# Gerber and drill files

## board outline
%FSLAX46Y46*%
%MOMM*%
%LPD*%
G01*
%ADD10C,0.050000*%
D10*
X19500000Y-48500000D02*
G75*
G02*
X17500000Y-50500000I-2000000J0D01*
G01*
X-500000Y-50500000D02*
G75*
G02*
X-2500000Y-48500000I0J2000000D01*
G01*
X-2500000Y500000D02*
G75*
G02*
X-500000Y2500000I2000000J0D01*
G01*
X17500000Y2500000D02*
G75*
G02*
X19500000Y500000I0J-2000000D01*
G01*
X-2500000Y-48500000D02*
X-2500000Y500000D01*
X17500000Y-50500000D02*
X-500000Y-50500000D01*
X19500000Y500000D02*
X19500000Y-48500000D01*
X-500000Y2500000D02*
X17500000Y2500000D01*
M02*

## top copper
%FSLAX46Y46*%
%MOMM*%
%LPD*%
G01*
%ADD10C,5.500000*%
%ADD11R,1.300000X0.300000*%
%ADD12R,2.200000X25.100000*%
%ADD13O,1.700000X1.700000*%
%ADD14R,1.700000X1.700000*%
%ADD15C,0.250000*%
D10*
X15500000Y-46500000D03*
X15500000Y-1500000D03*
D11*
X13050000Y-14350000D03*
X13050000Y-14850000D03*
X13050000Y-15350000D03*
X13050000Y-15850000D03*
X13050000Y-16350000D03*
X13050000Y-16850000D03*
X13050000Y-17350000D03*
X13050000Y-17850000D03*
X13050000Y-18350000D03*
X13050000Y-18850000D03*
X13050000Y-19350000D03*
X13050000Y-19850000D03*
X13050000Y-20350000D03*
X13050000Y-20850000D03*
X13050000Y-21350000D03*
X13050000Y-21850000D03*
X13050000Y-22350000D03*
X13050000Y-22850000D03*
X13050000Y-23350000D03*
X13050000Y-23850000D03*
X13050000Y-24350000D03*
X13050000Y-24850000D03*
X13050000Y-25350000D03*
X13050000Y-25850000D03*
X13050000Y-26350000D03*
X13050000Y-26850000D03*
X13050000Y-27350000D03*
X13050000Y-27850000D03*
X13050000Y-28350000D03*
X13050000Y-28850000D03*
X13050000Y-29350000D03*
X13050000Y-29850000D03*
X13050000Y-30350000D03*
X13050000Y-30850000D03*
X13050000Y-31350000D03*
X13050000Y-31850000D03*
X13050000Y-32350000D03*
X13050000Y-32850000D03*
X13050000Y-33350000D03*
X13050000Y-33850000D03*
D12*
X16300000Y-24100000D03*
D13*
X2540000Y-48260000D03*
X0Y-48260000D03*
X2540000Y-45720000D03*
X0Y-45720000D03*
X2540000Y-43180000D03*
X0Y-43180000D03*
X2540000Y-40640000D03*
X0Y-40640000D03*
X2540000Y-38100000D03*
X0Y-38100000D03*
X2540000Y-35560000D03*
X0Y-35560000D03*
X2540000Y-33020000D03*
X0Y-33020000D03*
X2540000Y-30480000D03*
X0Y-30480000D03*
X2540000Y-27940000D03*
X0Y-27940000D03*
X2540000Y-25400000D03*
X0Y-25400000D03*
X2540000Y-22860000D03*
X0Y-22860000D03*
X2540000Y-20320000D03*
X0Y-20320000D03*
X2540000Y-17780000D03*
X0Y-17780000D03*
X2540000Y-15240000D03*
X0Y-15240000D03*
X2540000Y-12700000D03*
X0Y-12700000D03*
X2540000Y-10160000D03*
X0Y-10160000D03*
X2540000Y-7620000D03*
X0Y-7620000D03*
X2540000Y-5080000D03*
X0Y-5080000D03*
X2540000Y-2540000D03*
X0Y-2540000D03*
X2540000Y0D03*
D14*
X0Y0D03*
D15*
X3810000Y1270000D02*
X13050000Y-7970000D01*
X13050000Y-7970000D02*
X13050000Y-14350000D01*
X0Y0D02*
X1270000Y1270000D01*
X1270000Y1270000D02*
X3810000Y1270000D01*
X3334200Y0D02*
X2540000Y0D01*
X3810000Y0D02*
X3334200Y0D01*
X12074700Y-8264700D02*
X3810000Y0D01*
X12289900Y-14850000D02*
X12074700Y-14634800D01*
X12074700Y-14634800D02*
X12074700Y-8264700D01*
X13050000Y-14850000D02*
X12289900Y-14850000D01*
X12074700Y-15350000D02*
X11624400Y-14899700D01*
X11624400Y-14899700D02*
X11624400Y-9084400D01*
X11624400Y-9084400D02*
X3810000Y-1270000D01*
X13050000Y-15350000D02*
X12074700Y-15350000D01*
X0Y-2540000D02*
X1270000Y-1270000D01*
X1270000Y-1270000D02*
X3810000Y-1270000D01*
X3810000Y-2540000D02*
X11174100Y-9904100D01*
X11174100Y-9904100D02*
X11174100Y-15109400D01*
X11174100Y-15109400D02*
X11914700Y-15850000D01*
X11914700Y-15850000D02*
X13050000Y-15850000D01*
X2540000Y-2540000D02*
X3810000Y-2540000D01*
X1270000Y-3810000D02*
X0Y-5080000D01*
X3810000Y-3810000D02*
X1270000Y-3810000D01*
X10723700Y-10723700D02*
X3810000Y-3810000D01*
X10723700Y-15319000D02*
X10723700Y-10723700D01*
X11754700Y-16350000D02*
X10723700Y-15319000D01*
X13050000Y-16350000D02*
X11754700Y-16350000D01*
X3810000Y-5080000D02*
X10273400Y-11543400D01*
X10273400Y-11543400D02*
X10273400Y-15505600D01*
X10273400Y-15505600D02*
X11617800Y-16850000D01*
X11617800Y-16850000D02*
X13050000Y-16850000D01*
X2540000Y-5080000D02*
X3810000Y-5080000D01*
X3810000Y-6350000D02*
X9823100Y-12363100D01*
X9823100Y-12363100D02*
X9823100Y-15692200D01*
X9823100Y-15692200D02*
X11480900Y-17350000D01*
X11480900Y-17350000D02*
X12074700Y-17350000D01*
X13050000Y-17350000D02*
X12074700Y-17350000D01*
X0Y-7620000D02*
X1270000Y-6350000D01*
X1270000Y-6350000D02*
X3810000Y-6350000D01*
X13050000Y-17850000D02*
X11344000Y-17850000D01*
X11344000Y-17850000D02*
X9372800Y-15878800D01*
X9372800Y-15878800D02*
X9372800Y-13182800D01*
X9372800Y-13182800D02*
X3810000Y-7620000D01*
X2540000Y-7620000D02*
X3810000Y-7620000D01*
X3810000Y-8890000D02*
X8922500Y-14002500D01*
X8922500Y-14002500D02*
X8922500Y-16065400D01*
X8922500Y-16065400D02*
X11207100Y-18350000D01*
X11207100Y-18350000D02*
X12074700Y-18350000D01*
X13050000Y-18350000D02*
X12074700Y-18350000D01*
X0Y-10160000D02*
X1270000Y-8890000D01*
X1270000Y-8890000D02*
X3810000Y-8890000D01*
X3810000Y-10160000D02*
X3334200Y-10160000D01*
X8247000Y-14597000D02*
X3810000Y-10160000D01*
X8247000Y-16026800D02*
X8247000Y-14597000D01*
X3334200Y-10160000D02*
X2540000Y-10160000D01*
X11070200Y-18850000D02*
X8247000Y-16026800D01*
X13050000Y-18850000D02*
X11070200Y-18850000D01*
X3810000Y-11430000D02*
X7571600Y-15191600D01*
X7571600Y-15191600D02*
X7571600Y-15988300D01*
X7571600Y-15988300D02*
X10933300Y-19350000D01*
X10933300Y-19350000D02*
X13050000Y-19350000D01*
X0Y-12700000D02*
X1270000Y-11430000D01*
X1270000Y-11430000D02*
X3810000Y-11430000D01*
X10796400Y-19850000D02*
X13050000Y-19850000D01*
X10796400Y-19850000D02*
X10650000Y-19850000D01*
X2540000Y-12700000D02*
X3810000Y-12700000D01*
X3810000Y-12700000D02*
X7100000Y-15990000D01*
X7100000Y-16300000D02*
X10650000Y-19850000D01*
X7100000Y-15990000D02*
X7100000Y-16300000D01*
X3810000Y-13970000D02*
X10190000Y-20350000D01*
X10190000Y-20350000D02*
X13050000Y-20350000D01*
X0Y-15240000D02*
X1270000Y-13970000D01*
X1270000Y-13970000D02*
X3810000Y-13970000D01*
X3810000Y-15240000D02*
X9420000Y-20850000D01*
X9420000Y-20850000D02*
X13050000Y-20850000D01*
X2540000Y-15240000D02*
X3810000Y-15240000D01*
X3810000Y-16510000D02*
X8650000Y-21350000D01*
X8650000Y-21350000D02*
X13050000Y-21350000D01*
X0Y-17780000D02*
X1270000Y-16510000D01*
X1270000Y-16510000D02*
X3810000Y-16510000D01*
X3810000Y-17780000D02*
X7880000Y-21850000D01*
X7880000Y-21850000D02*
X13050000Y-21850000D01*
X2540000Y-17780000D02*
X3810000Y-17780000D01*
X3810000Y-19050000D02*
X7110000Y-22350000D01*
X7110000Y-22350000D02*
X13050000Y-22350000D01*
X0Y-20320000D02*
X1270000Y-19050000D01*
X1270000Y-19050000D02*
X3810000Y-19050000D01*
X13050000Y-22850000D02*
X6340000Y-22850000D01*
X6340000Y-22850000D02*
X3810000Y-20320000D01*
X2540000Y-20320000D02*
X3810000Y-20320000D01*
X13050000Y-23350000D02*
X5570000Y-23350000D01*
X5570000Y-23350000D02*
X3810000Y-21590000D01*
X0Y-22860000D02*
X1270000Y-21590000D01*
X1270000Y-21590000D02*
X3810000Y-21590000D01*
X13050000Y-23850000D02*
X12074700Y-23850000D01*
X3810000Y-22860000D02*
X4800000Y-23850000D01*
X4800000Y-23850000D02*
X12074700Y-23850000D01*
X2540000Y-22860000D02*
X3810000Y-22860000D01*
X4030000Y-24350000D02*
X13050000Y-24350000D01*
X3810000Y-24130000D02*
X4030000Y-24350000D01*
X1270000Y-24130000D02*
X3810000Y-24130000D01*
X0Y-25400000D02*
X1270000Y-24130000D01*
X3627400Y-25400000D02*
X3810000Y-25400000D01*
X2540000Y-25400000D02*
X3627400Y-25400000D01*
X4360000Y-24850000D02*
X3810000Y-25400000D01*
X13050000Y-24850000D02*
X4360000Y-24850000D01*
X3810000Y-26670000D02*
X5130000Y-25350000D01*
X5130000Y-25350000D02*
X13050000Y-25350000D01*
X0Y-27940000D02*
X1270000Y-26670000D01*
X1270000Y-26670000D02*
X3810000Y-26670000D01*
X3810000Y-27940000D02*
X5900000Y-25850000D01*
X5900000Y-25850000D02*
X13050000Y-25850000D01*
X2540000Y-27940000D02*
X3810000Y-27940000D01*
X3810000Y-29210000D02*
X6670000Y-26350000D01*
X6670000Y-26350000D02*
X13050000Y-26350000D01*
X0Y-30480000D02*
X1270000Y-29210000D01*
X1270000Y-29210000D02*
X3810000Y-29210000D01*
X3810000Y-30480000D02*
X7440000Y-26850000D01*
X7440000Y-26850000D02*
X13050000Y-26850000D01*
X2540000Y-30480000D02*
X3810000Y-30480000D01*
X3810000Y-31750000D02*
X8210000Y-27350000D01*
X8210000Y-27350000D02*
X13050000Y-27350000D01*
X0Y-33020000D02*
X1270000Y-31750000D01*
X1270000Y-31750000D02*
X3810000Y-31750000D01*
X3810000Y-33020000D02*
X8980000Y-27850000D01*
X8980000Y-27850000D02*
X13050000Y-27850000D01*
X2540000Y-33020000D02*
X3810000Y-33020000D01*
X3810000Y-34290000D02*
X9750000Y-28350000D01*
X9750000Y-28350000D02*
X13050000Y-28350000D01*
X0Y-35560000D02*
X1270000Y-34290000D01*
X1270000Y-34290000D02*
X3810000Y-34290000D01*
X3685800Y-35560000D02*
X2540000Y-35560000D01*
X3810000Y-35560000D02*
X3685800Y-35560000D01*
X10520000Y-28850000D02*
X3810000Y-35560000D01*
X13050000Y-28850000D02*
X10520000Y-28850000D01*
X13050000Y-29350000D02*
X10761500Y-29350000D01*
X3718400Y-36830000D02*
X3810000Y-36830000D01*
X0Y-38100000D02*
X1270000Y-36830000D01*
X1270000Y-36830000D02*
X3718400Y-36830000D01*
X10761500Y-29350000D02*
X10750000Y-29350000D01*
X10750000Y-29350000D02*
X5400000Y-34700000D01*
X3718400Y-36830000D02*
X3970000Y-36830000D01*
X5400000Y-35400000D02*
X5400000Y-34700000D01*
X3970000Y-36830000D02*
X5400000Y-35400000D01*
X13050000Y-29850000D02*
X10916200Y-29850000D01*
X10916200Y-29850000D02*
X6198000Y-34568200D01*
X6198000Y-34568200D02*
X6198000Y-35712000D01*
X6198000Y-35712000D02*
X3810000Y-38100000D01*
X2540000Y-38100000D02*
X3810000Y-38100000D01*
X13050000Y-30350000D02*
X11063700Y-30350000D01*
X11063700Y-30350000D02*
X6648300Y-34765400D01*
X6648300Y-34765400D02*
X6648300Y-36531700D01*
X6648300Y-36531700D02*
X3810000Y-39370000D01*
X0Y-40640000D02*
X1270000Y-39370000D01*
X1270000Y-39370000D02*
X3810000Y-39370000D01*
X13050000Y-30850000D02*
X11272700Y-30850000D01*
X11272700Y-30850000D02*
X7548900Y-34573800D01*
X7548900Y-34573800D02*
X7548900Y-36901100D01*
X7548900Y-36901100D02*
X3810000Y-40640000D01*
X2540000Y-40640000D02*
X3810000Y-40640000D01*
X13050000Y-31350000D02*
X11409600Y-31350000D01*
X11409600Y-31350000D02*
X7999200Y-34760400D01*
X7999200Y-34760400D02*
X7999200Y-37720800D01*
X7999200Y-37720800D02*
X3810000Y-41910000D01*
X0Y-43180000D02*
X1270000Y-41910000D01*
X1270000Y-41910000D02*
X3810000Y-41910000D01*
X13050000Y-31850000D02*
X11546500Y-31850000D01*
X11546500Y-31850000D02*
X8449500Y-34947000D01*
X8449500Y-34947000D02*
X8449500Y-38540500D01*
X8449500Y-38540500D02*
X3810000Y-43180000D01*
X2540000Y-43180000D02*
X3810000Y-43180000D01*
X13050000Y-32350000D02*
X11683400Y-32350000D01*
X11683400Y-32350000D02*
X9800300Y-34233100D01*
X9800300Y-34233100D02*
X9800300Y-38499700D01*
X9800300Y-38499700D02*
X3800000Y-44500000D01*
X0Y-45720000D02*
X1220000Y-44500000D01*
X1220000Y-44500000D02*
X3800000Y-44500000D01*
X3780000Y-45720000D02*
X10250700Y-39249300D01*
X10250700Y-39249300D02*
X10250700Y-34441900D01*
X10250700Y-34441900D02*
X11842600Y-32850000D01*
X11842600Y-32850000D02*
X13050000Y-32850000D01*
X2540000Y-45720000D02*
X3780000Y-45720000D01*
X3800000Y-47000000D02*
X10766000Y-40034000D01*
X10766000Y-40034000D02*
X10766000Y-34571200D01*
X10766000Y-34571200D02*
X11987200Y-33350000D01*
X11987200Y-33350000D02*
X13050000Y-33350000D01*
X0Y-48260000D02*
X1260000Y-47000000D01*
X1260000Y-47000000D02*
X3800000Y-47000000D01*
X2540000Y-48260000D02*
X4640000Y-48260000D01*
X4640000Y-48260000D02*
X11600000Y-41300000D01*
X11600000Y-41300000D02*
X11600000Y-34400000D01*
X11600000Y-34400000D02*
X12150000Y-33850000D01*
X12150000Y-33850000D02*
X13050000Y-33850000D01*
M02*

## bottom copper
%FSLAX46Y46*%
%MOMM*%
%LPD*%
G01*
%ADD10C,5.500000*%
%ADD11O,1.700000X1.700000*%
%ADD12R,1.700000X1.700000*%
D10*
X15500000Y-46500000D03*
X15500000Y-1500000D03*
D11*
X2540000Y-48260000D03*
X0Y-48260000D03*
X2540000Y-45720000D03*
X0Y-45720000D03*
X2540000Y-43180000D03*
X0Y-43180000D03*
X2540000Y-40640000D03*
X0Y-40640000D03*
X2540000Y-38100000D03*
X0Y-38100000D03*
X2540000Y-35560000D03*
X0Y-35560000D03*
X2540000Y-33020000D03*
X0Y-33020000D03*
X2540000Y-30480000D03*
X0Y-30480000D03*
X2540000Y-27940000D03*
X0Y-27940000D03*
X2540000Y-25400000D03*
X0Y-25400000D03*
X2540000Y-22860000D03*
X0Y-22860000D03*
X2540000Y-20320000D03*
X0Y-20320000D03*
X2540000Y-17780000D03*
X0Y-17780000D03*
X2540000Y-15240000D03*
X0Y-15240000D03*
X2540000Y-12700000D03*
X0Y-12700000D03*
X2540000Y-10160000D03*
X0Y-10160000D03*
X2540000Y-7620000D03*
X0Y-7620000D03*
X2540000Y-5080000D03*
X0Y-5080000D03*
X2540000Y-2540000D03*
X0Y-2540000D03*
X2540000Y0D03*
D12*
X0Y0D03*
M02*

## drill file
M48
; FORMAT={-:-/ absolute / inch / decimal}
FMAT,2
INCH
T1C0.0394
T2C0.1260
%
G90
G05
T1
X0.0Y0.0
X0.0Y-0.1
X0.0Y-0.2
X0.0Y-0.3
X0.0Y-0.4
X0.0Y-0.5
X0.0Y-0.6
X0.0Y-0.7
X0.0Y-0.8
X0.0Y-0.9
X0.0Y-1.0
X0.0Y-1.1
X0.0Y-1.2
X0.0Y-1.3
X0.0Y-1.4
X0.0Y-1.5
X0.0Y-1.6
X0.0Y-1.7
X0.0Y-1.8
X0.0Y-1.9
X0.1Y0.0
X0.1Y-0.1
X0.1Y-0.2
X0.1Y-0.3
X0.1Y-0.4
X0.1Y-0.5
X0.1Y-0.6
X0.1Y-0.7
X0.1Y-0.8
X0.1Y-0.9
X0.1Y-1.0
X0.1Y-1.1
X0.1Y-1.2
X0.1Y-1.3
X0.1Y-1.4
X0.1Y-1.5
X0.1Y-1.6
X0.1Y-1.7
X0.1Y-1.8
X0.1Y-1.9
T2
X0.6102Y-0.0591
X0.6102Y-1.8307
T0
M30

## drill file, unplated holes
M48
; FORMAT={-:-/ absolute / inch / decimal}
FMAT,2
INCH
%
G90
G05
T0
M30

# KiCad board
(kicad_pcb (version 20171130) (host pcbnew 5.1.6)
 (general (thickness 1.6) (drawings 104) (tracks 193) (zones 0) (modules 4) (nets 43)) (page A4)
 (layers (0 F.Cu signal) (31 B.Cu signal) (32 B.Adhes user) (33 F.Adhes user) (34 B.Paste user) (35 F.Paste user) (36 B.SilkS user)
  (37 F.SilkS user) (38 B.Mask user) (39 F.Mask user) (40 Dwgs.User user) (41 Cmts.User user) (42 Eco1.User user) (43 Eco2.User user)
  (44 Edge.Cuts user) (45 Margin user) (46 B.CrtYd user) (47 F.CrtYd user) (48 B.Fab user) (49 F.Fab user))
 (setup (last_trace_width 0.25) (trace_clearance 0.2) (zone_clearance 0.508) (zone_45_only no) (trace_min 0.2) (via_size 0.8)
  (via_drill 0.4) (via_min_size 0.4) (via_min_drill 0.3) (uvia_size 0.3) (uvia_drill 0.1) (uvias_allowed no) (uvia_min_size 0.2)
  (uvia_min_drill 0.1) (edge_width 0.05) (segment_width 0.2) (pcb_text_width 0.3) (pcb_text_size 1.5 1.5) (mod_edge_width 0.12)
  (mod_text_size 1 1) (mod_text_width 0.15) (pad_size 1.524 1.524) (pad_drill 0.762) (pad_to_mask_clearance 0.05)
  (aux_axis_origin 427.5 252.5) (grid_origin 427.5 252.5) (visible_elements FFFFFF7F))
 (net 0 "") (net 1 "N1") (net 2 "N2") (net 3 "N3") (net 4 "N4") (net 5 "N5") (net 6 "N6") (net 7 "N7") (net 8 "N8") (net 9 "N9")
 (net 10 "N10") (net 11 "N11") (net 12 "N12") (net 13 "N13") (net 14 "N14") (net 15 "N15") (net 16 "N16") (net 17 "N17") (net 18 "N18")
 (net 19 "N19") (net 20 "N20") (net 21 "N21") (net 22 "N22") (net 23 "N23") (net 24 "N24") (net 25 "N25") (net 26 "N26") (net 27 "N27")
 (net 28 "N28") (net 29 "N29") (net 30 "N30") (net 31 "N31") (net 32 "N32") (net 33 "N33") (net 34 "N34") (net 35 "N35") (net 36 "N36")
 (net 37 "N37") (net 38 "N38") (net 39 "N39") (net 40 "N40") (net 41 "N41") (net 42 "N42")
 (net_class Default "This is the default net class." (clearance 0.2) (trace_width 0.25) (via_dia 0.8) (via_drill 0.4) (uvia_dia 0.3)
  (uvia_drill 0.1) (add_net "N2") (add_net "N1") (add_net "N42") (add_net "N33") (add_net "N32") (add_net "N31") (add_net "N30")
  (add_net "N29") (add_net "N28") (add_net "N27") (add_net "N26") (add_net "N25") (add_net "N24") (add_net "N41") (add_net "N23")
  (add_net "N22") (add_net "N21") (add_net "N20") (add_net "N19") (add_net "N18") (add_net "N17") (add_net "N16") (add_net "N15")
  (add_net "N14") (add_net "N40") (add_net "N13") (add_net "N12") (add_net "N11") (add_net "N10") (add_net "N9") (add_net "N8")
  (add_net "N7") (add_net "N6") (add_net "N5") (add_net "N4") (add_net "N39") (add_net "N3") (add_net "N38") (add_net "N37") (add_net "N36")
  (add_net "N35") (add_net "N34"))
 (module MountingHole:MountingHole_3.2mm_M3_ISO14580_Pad (layer F.Cu) (at 443 299)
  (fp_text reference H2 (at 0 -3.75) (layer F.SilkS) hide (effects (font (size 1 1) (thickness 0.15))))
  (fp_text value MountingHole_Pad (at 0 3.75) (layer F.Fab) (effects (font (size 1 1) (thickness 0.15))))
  (pad 1 thru_hole circle (at 0 0) (size 5.5 5.5) (drill 3.2) (layers *.Cu *.Mask) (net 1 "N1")))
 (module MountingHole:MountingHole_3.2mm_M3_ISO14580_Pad (layer F.Cu) (at 443 254)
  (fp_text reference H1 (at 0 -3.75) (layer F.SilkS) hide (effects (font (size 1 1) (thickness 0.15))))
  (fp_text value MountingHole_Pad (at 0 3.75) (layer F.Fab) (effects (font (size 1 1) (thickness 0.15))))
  (pad 1 thru_hole circle (at 0 0) (size 5.5 5.5) (drill 3.2) (layers *.Cu *.Mask) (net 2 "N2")))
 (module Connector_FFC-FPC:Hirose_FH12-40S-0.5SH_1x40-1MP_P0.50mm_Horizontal (layer F.Cu) (at 442.4 276.6 90)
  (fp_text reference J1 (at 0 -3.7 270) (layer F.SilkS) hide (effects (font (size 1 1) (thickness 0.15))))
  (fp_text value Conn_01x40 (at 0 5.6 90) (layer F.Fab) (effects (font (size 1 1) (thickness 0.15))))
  (pad 40 smd rect (at 9.75 -1.85 90) (size 0.3 1.3) (layers F.Cu F.Paste F.Mask) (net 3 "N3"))
  (pad 39 smd rect (at 9.25 -1.85 90) (size 0.3 1.3) (layers F.Cu F.Paste F.Mask) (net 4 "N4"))
  (pad 38 smd rect (at 8.75 -1.85 90) (size 0.3 1.3) (layers F.Cu F.Paste F.Mask) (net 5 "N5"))
  (pad 37 smd rect (at 8.25 -1.85 90) (size 0.3 1.3) (layers F.Cu F.Paste F.Mask) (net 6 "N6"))
  (pad 36 smd rect (at 7.75 -1.85 90) (size 0.3 1.3) (layers F.Cu F.Paste F.Mask) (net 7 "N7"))
  (pad 35 smd rect (at 7.25 -1.85 90) (size 0.3 1.3) (layers F.Cu F.Paste F.Mask) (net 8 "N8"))
  (pad 34 smd rect (at 6.75 -1.85 90) (size 0.3 1.3) (layers F.Cu F.Paste F.Mask) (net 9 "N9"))
  (pad 33 smd rect (at 6.25 -1.85 90) (size 0.3 1.3) (layers F.Cu F.Paste F.Mask) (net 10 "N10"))
  (pad 32 smd rect (at 5.75 -1.85 90) (size 0.3 1.3) (layers F.Cu F.Paste F.Mask) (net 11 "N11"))
  (pad 31 smd rect (at 5.25 -1.85 90) (size 0.3 1.3) (layers F.Cu F.Paste F.Mask) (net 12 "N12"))
  (pad 30 smd rect (at 4.75 -1.85 90) (size 0.3 1.3) (layers F.Cu F.Paste F.Mask) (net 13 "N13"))
  (pad 29 smd rect (at 4.25 -1.85 90) (size 0.3 1.3) (layers F.Cu F.Paste F.Mask) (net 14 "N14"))
  (pad 28 smd rect (at 3.75 -1.85 90) (size 0.3 1.3) (layers F.Cu F.Paste F.Mask) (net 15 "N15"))
  (pad 27 smd rect (at 3.25 -1.85 90) (size 0.3 1.3) (layers F.Cu F.Paste F.Mask) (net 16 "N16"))
  (pad 26 smd rect (at 2.75 -1.85 90) (size 0.3 1.3) (layers F.Cu F.Paste F.Mask) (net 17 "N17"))
  (pad 25 smd rect (at 2.25 -1.85 90) (size 0.3 1.3) (layers F.Cu F.Paste F.Mask) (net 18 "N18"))
  (pad 24 smd rect (at 1.75 -1.85 90) (size 0.3 1.3) (layers F.Cu F.Paste F.Mask) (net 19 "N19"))
  (pad 23 smd rect (at 1.25 -1.85 90) (size 0.3 1.3) (layers F.Cu F.Paste F.Mask) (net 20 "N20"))
  (pad 22 smd rect (at 0.75 -1.85 90) (size 0.3 1.3) (layers F.Cu F.Paste F.Mask) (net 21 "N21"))
  (pad 21 smd rect (at 0.25 -1.85 90) (size 0.3 1.3) (layers F.Cu F.Paste F.Mask) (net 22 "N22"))
  (pad 20 smd rect (at -0.25 -1.85 90) (size 0.3 1.3) (layers F.Cu F.Paste F.Mask) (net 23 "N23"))
  (pad 19 smd rect (at -0.75 -1.85 90) (size 0.3 1.3) (layers F.Cu F.Paste F.Mask) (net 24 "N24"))
  (pad 18 smd rect (at -1.25 -1.85 90) (size 0.3 1.3) (layers F.Cu F.Paste F.Mask) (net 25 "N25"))
  (pad 17 smd rect (at -1.75 -1.85 90) (size 0.3 1.3) (layers F.Cu F.Paste F.Mask) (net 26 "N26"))
  (pad 16 smd rect (at -2.25 -1.85 90) (size 0.3 1.3) (layers F.Cu F.Paste F.Mask) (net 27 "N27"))
  (pad 15 smd rect (at -2.75 -1.85 90) (size 0.3 1.3) (layers F.Cu F.Paste F.Mask) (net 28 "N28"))
  (pad 14 smd rect (at -3.25 -1.85 90) (size 0.3 1.3) (layers F.Cu F.Paste F.Mask) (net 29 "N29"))
  (pad 13 smd rect (at -3.75 -1.85 90) (size 0.3 1.3) (layers F.Cu F.Paste F.Mask) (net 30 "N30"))
  (pad 12 smd rect (at -4.25 -1.85 90) (size 0.3 1.3) (layers F.Cu F.Paste F.Mask) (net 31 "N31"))
  (pad 11 smd rect (at -4.75 -1.85 90) (size 0.3 1.3) (layers F.Cu F.Paste F.Mask) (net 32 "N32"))
  (pad 10 smd rect (at -5.25 -1.85 90) (size 0.3 1.3) (layers F.Cu F.Paste F.Mask) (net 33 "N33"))
  (pad 9 smd rect (at -5.75 -1.85 90) (size 0.3 1.3) (layers F.Cu F.Paste F.Mask) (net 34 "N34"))
  (pad 8 smd rect (at -6.25 -1.85 90) (size 0.3 1.3) (layers F.Cu F.Paste F.Mask) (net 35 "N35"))
  (pad 7 smd rect (at -6.75 -1.85 90) (size 0.3 1.3) (layers F.Cu F.Paste F.Mask) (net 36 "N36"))
  (pad 6 smd rect (at -7.25 -1.85 90) (size 0.3 1.3) (layers F.Cu F.Paste F.Mask) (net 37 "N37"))
  (pad 5 smd rect (at -7.75 -1.85 90) (size 0.3 1.3) (layers F.Cu F.Paste F.Mask) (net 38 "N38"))
  (pad 4 smd rect (at -8.25 -1.85 90) (size 0.3 1.3) (layers F.Cu F.Paste F.Mask) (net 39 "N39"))
  (pad 3 smd rect (at -8.75 -1.85 90) (size 0.3 1.3) (layers F.Cu F.Paste F.Mask) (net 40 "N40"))
  (pad 2 smd rect (at -9.25 -1.85 90) (size 0.3 1.3) (layers F.Cu F.Paste F.Mask) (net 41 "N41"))
  (pad 1 smd rect (at -9.75 -1.85 90) (size 0.3 1.3) (layers F.Cu F.Paste F.Mask) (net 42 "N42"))
  (pad MP smd rect (at 0 1.4 90) (size 25.1 2.2) (layers F.Cu F.Paste F.Mask)))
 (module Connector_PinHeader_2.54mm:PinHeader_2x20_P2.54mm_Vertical (layer F.Cu) (at 427.5 252.5)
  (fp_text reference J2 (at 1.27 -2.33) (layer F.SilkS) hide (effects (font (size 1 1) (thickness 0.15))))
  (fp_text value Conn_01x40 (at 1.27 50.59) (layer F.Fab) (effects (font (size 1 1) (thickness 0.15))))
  (pad 40 thru_hole oval (at 2.54 48.26) (size 1.7 1.7) (drill 1) (layers *.Cu *.Mask) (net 42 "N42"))
  (pad 39 thru_hole oval (at 0 48.26) (size 1.7 1.7) (drill 1) (layers *.Cu *.Mask) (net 41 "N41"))
  (pad 38 thru_hole oval (at 2.54 45.72) (size 1.7 1.7) (drill 1) (layers *.Cu *.Mask) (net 40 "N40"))
  (pad 37 thru_hole oval (at 0 45.72) (size 1.7 1.7) (drill 1) (layers *.Cu *.Mask) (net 39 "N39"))
  (pad 36 thru_hole oval (at 2.54 43.18) (size 1.7 1.7) (drill 1) (layers *.Cu *.Mask) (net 38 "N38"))
  (pad 35 thru_hole oval (at 0 43.18) (size 1.7 1.7) (drill 1) (layers *.Cu *.Mask) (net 37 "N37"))
  (pad 34 thru_hole oval (at 2.54 40.64) (size 1.7 1.7) (drill 1) (layers *.Cu *.Mask) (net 36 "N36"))
  (pad 33 thru_hole oval (at 0 40.64) (size 1.7 1.7) (drill 1) (layers *.Cu *.Mask) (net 35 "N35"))
  (pad 32 thru_hole oval (at 2.54 38.1) (size 1.7 1.7) (drill 1) (layers *.Cu *.Mask) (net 34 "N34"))
  (pad 31 thru_hole oval (at 0 38.1) (size 1.7 1.7) (drill 1) (layers *.Cu *.Mask) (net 33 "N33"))
  (pad 30 thru_hole oval (at 2.54 35.56) (size 1.7 1.7) (drill 1) (layers *.Cu *.Mask) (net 32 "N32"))
  (pad 29 thru_hole oval (at 0 35.56) (size 1.7 1.7) (drill 1) (layers *.Cu *.Mask) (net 31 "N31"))
  (pad 28 thru_hole oval (at 2.54 33.02) (size 1.7 1.7) (drill 1) (layers *.Cu *.Mask) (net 30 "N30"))
  (pad 27 thru_hole oval (at 0 33.02) (size 1.7 1.7) (drill 1) (layers *.Cu *.Mask) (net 29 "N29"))
  (pad 26 thru_hole oval (at 2.54 30.48) (size 1.7 1.7) (drill 1) (layers *.Cu *.Mask) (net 28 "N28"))
  (pad 25 thru_hole oval (at 0 30.48) (size 1.7 1.7) (drill 1) (layers *.Cu *.Mask) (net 27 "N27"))
  (pad 24 thru_hole oval (at 2.54 27.94) (size 1.7 1.7) (drill 1) (layers *.Cu *.Mask) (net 26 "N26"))
  (pad 23 thru_hole oval (at 0 27.94) (size 1.7 1.7) (drill 1) (layers *.Cu *.Mask) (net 25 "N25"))
  (pad 22 thru_hole oval (at 2.54 25.4) (size 1.7 1.7) (drill 1) (layers *.Cu *.Mask) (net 24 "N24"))
  (pad 21 thru_hole oval (at 0 25.4) (size 1.7 1.7) (drill 1) (layers *.Cu *.Mask) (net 23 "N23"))
  (pad 20 thru_hole oval (at 2.54 22.86) (size 1.7 1.7) (drill 1) (layers *.Cu *.Mask) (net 22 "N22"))
  (pad 19 thru_hole oval (at 0 22.86) (size 1.7 1.7) (drill 1) (layers *.Cu *.Mask) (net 21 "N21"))
  (pad 18 thru_hole oval (at 2.54 20.32) (size 1.7 1.7) (drill 1) (layers *.Cu *.Mask) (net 20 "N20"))
  (pad 17 thru_hole oval (at 0 20.32) (size 1.7 1.7) (drill 1) (layers *.Cu *.Mask) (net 19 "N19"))
  (pad 16 thru_hole oval (at 2.54 17.78) (size 1.7 1.7) (drill 1) (layers *.Cu *.Mask) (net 18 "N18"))
  (pad 15 thru_hole oval (at 0 17.78) (size 1.7 1.7) (drill 1) (layers *.Cu *.Mask) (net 17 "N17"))
  (pad 14 thru_hole oval (at 2.54 15.24) (size 1.7 1.7) (drill 1) (layers *.Cu *.Mask) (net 16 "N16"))
  (pad 13 thru_hole oval (at 0 15.24) (size 1.7 1.7) (drill 1) (layers *.Cu *.Mask) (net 15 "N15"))
  (pad 12 thru_hole oval (at 2.54 12.7) (size 1.7 1.7) (drill 1) (layers *.Cu *.Mask) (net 14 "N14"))
  (pad 11 thru_hole oval (at 0 12.7) (size 1.7 1.7) (drill 1) (layers *.Cu *.Mask) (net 13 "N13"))
  (pad 10 thru_hole oval (at 2.54 10.16) (size 1.7 1.7) (drill 1) (layers *.Cu *.Mask) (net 12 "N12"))
  (pad 9 thru_hole oval (at 0 10.16) (size 1.7 1.7) (drill 1) (layers *.Cu *.Mask) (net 11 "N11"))
  (pad 8 thru_hole oval (at 2.54 7.62) (size 1.7 1.7) (drill 1) (layers *.Cu *.Mask) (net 10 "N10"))
  (pad 7 thru_hole oval (at 0 7.62) (size 1.7 1.7) (drill 1) (layers *.Cu *.Mask) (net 9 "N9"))
  (pad 6 thru_hole oval (at 2.54 5.08) (size 1.7 1.7) (drill 1) (layers *.Cu *.Mask) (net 8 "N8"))
  (pad 5 thru_hole oval (at 0 5.08) (size 1.7 1.7) (drill 1) (layers *.Cu *.Mask) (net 7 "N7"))
  (pad 4 thru_hole oval (at 2.54 2.54) (size 1.7 1.7) (drill 1) (layers *.Cu *.Mask) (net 6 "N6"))
  (pad 3 thru_hole oval (at 0 2.54) (size 1.7 1.7) (drill 1) (layers *.Cu *.Mask) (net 5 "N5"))
  (pad 2 thru_hole oval (at 2.54 0) (size 1.7 1.7) (drill 1) (layers *.Cu *.Mask) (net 4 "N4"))
  (pad 1 thru_hole rect (at 0 0) (size 1.7 1.7) (drill 1) (layers *.Cu *.Mask) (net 3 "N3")))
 (gr_arc (start 445 301) (end 445 303) (angle -90) (layer Edge.Cuts) (width 0.05))
 (gr_arc (start 427 301) (end 425 301) (angle -90) (layer Edge.Cuts) (width 0.05))
 (gr_arc (start 427 252) (end 427 250) (angle -90) (layer Edge.Cuts) (width 0.05))
 (gr_arc (start 445 252) (end 447 252) (angle -90) (layer Edge.Cuts) (width 0.05))
 (gr_line (start 425 301) (end 425 252) (layer Edge.Cuts) (width 0.05))
 (gr_line (start 445 303) (end 427 303) (layer Edge.Cuts) (width 0.05))
 (gr_line (start 447 252) (end 447 301) (layer Edge.Cuts) (width 0.05))
 (gr_line (start 427 250) (end 445 250) (layer Edge.Cuts) (width 0.05))
 (segment (start 431.31 251.23) (end 440.55 260.47) (width 0.25) (layer F.Cu) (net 3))
 (segment (start 440.55 260.47) (end 440.55 266.85) (width 0.25) (layer F.Cu) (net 3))
 (segment (start 427.5 252.5) (end 428.77 251.23) (width 0.25) (layer F.Cu) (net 3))
 (segment (start 428.77 251.23) (end 431.31 251.23) (width 0.25) (layer F.Cu) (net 3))
 (segment (start 430.8342 252.5) (end 430.04 252.5) (width 0.25) (layer F.Cu) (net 4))
 (segment (start 431.31 252.5) (end 430.8342 252.5) (width 0.25) (layer F.Cu) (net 4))
 (segment (start 439.5747 260.7647) (end 431.31 252.5) (width 0.25) (layer F.Cu) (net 4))
 (segment (start 439.7899 267.35) (end 439.5747 267.1348) (width 0.25) (layer F.Cu) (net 4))
 (segment (start 439.5747 267.1348) (end 439.5747 260.7647) (width 0.25) (layer F.Cu) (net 4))
 (segment (start 440.55 267.35) (end 439.7899 267.35) (width 0.25) (layer F.Cu) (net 4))
 (segment (start 439.5747 267.85) (end 439.1244 267.3997) (width 0.25) (layer F.Cu) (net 5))
 (segment (start 439.1244 267.3997) (end 439.1244 261.5844) (width 0.25) (layer F.Cu) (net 5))
 (segment (start 439.1244 261.5844) (end 431.31 253.77) (width 0.25) (layer F.Cu) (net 5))
 (segment (start 440.55 267.85) (end 439.5747 267.85) (width 0.25) (layer F.Cu) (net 5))
 (segment (start 427.5 255.04) (end 428.77 253.77) (width 0.25) (layer F.Cu) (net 5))
 (segment (start 428.77 253.77) (end 431.31 253.77) (width 0.25) (layer F.Cu) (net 5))
 (segment (start 431.31 255.04) (end 438.6741 262.4041) (width 0.25) (layer F.Cu) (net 6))
 (segment (start 438.6741 262.4041) (end 438.6741 267.6094) (width 0.25) (layer F.Cu) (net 6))
 (segment (start 438.6741 267.6094) (end 439.4147 268.35) (width 0.25) (layer F.Cu) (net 6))
 (segment (start 439.4147 268.35) (end 440.55 268.35) (width 0.25) (layer F.Cu) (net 6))
 (segment (start 430.04 255.04) (end 431.31 255.04) (width 0.25) (layer F.Cu) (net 6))
 (segment (start 428.77 256.31) (end 427.5 257.58) (width 0.25) (layer F.Cu) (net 7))
 (segment (start 431.31 256.31) (end 428.77 256.31) (width 0.25) (layer F.Cu) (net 7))
 (segment (start 438.2237 263.2237) (end 431.31 256.31) (width 0.25) (layer F.Cu) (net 7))
 (segment (start 438.2237 267.819) (end 438.2237 263.2237) (width 0.25) (layer F.Cu) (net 7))
 (segment (start 439.2547 268.85) (end 438.2237 267.819) (width 0.25) (layer F.Cu) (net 7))
 (segment (start 440.55 268.85) (end 439.2547 268.85) (width 0.25) (layer F.Cu) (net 7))
 (segment (start 431.31 257.58) (end 437.7734 264.0434) (width 0.25) (layer F.Cu) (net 8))
 (segment (start 437.7734 264.0434) (end 437.7734 268.0056) (width 0.25) (layer F.Cu) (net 8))
 (segment (start 437.7734 268.0056) (end 439.1178 269.35) (width 0.25) (layer F.Cu) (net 8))
 (segment (start 439.1178 269.35) (end 440.55 269.35) (width 0.25) (layer F.Cu) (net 8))
 (segment (start 430.04 257.58) (end 431.31 257.58) (width 0.25) (layer F.Cu) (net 8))
 (segment (start 431.31 258.85) (end 437.3231 264.8631) (width 0.25) (layer F.Cu) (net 9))
 (segment (start 437.3231 264.8631) (end 437.3231 268.1922) (width 0.25) (layer F.Cu) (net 9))
 (segment (start 437.3231 268.1922) (end 438.9809 269.85) (width 0.25) (layer F.Cu) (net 9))
 (segment (start 438.9809 269.85) (end 439.5747 269.85) (width 0.25) (layer F.Cu) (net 9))
 (segment (start 440.55 269.85) (end 439.5747 269.85) (width 0.25) (layer F.Cu) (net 9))
 (segment (start 427.5 260.12) (end 428.77 258.85) (width 0.25) (layer F.Cu) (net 9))
 (segment (start 428.77 258.85) (end 431.31 258.85) (width 0.25) (layer F.Cu) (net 9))
 (segment (start 440.55 270.35) (end 438.844 270.35) (width 0.25) (layer F.Cu) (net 10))
 (segment (start 438.844 270.35) (end 436.8728 268.3788) (width 0.25) (layer F.Cu) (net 10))
 (segment (start 436.8728 268.3788) (end 436.8728 265.6828) (width 0.25) (layer F.Cu) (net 10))
 (segment (start 436.8728 265.6828) (end 431.31 260.12) (width 0.25) (layer F.Cu) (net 10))
 (segment (start 430.04 260.12) (end 431.31 260.12) (width 0.25) (layer F.Cu) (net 10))
 (segment (start 431.31 261.39) (end 436.4225 266.5025) (width 0.25) (layer F.Cu) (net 11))
 (segment (start 436.4225 266.5025) (end 436.4225 268.5654) (width 0.25) (layer F.Cu) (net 11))
 (segment (start 436.4225 268.5654) (end 438.7071 270.85) (width 0.25) (layer F.Cu) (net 11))
 (segment (start 438.7071 270.85) (end 439.5747 270.85) (width 0.25) (layer F.Cu) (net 11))
 (segment (start 440.55 270.85) (end 439.5747 270.85) (width 0.25) (layer F.Cu) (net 11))
 (segment (start 427.5 262.66) (end 428.77 261.39) (width 0.25) (layer F.Cu) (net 11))
 (segment (start 428.77 261.39) (end 431.31 261.39) (width 0.25) (layer F.Cu) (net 11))
 (segment (start 431.31 262.66) (end 430.8342 262.66) (width 0.25) (layer F.Cu) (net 12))
 (segment (start 435.747 267.097) (end 431.31 262.66) (width 0.25) (layer F.Cu) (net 12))
 (segment (start 435.747 268.5268) (end 435.747 267.097) (width 0.25) (layer F.Cu) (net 12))
 (segment (start 430.8342 262.66) (end 430.04 262.66) (width 0.25) (layer F.Cu) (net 12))
 (segment (start 438.5702 271.35) (end 435.747 268.5268) (width 0.25) (layer F.Cu) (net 12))
 (segment (start 440.55 271.35) (end 438.5702 271.35) (width 0.25) (layer F.Cu) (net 12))
 (segment (start 431.31 263.93) (end 435.0716 267.6916) (width 0.25) (layer F.Cu) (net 13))
 (segment (start 435.0716 267.6916) (end 435.0716 268.4883) (width 0.25) (layer F.Cu) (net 13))
 (segment (start 435.0716 268.4883) (end 438.4333 271.85) (width 0.25) (layer F.Cu) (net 13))
 (segment (start 438.4333 271.85) (end 440.55 271.85) (width 0.25) (layer F.Cu) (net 13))
 (segment (start 427.5 265.2) (end 428.77 263.93) (width 0.25) (layer F.Cu) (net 13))
 (segment (start 428.77 263.93) (end 431.31 263.93) (width 0.25) (layer F.Cu) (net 13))
 (segment (start 438.2964 272.35) (end 440.55 272.35) (width 0.25) (layer F.Cu) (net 14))
 (segment (start 438.2964 272.35) (end 438.15 272.35) (width 0.25) (layer F.Cu) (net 14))
 (segment (start 430.04 265.2) (end 431.31 265.2) (width 0.25) (layer F.Cu) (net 14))
 (segment (start 431.31 265.2) (end 434.6 268.49) (width 0.25) (layer F.Cu) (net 14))
 (segment (start 434.6 268.8) (end 438.15 272.35) (width 0.25) (layer F.Cu) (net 14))
 (segment (start 434.6 268.49) (end 434.6 268.8) (width 0.25) (layer F.Cu) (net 14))
 (segment (start 431.31 266.47) (end 437.69 272.85) (width 0.25) (layer F.Cu) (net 15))
 (segment (start 437.69 272.85) (end 440.55 272.85) (width 0.25) (layer F.Cu) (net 15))
 (segment (start 427.5 267.74) (end 428.77 266.47) (width 0.25) (layer F.Cu) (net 15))
 (segment (start 428.77 266.47) (end 431.31 266.47) (width 0.25) (layer F.Cu) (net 15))
 (segment (start 431.31 267.74) (end 436.92 273.35) (width 0.25) (layer F.Cu) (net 16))
 (segment (start 436.92 273.35) (end 440.55 273.35) (width 0.25) (layer F.Cu) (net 16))
 (segment (start 430.04 267.74) (end 431.31 267.74) (width 0.25) (layer F.Cu) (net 16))
 (segment (start 431.31 269.01) (end 436.15 273.85) (width 0.25) (layer F.Cu) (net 17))
 (segment (start 436.15 273.85) (end 440.55 273.85) (width 0.25) (layer F.Cu) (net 17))
 (segment (start 427.5 270.28) (end 428.77 269.01) (width 0.25) (layer F.Cu) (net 17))
 (segment (start 428.77 269.01) (end 431.31 269.01) (width 0.25) (layer F.Cu) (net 17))
 (segment (start 431.31 270.28) (end 435.38 274.35) (width 0.25) (layer F.Cu) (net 18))
 (segment (start 435.38 274.35) (end 440.55 274.35) (width 0.25) (layer F.Cu) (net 18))
 (segment (start 430.04 270.28) (end 431.31 270.28) (width 0.25) (layer F.Cu) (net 18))
 (segment (start 431.31 271.55) (end 434.61 274.85) (width 0.25) (layer F.Cu) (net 19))
 (segment (start 434.61 274.85) (end 440.55 274.85) (width 0.25) (layer F.Cu) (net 19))
 (segment (start 427.5 272.82) (end 428.77 271.55) (width 0.25) (layer F.Cu) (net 19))
 (segment (start 428.77 271.55) (end 431.31 271.55) (width 0.25) (layer F.Cu) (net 19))
 (segment (start 440.55 275.35) (end 433.84 275.35) (width 0.25) (layer F.Cu) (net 20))
 (segment (start 433.84 275.35) (end 431.31 272.82) (width 0.25) (layer F.Cu) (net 20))
 (segment (start 430.04 272.82) (end 431.31 272.82) (width 0.25) (layer F.Cu) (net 20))
 (segment (start 440.55 275.85) (end 433.07 275.85) (width 0.25) (layer F.Cu) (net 21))
 (segment (start 433.07 275.85) (end 431.31 274.09) (width 0.25) (layer F.Cu) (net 21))
 (segment (start 427.5 275.36) (end 428.77 274.09) (width 0.25) (layer F.Cu) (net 21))
 (segment (start 428.77 274.09) (end 431.31 274.09) (width 0.25) (layer F.Cu) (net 21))
 (segment (start 440.55 276.35) (end 439.5747 276.35) (width 0.25) (layer F.Cu) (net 22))
 (segment (start 431.31 275.36) (end 432.3 276.35) (width 0.25) (layer F.Cu) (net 22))
 (segment (start 432.3 276.35) (end 439.5747 276.35) (width 0.25) (layer F.Cu) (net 22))
 (segment (start 430.04 275.36) (end 431.31 275.36) (width 0.25) (layer F.Cu) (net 22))
 (segment (start 431.53 276.85) (end 440.55 276.85) (width 0.25) (layer F.Cu) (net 23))
 (segment (start 431.31 276.63) (end 431.53 276.85) (width 0.25) (layer F.Cu) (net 23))
 (segment (start 428.77 276.63) (end 431.31 276.63) (width 0.25) (layer F.Cu) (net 23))
 (segment (start 427.5 277.9) (end 428.77 276.63) (width 0.25) (layer F.Cu) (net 23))
 (segment (start 431.1274 277.9) (end 431.31 277.9) (width 0.25) (layer F.Cu) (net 24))
 (segment (start 430.04 277.9) (end 431.1274 277.9) (width 0.25) (layer F.Cu) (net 24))
 (segment (start 431.86 277.35) (end 431.31 277.9) (width 0.25) (layer F.Cu) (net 24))
 (segment (start 440.55 277.35) (end 431.86 277.35) (width 0.25) (layer F.Cu) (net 24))
 (segment (start 431.31 279.17) (end 432.63 277.85) (width 0.25) (layer F.Cu) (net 25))
 (segment (start 432.63 277.85) (end 440.55 277.85) (width 0.25) (layer F.Cu) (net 25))
 (segment (start 427.5 280.44) (end 428.77 279.17) (width 0.25) (layer F.Cu) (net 25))
 (segment (start 428.77 279.17) (end 431.31 279.17) (width 0.25) (layer F.Cu) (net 25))
 (segment (start 431.31 280.44) (end 433.4 278.35) (width 0.25) (layer F.Cu) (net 26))
 (segment (start 433.4 278.35) (end 440.55 278.35) (width 0.25) (layer F.Cu) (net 26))
 (segment (start 430.04 280.44) (end 431.31 280.44) (width 0.25) (layer F.Cu) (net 26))
 (segment (start 431.31 281.71) (end 434.17 278.85) (width 0.25) (layer F.Cu) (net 27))
 (segment (start 434.17 278.85) (end 440.55 278.85) (width 0.25) (layer F.Cu) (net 27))
 (segment (start 427.5 282.98) (end 428.77 281.71) (width 0.25) (layer F.Cu) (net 27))
 (segment (start 428.77 281.71) (end 431.31 281.71) (width 0.25) (layer F.Cu) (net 27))
 (segment (start 431.31 282.98) (end 434.94 279.35) (width 0.25) (layer F.Cu) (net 28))
 (segment (start 434.94 279.35) (end 440.55 279.35) (width 0.25) (layer F.Cu) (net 28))
 (segment (start 430.04 282.98) (end 431.31 282.98) (width 0.25) (layer F.Cu) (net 28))
 (segment (start 431.31 284.25) (end 435.71 279.85) (width 0.25) (layer F.Cu) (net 29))
 (segment (start 435.71 279.85) (end 440.55 279.85) (width 0.25) (layer F.Cu) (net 29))
 (segment (start 427.5 285.52) (end 428.77 284.25) (width 0.25) (layer F.Cu) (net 29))
 (segment (start 428.77 284.25) (end 431.31 284.25) (width 0.25) (layer F.Cu) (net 29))
 (segment (start 431.31 285.52) (end 436.48 280.35) (width 0.25) (layer F.Cu) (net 30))
 (segment (start 436.48 280.35) (end 440.55 280.35) (width 0.25) (layer F.Cu) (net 30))
 (segment (start 430.04 285.52) (end 431.31 285.52) (width 0.25) (layer F.Cu) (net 30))
 (segment (start 431.31 286.79) (end 437.25 280.85) (width 0.25) (layer F.Cu) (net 31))
 (segment (start 437.25 280.85) (end 440.55 280.85) (width 0.25) (layer F.Cu) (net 31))
 (segment (start 427.5 288.06) (end 428.77 286.79) (width 0.25) (layer F.Cu) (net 31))
 (segment (start 428.77 286.79) (end 431.31 286.79) (width 0.25) (layer F.Cu) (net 31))
 (segment (start 431.1858 288.06) (end 430.04 288.06) (width 0.25) (layer F.Cu) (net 32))
 (segment (start 431.31 288.06) (end 431.1858 288.06) (width 0.25) (layer F.Cu) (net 32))
 (segment (start 438.02 281.35) (end 431.31 288.06) (width 0.25) (layer F.Cu) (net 32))
 (segment (start 440.55 281.35) (end 438.02 281.35) (width 0.25) (layer F.Cu) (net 32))
 (segment (start 440.55 281.85) (end 438.2615 281.85) (width 0.25) (layer F.Cu) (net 33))
 (segment (start 431.2184 289.33) (end 431.31 289.33) (width 0.25) (layer F.Cu) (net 33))
 (segment (start 427.5 290.6) (end 428.77 289.33) (width 0.25) (layer F.Cu) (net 33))
 (segment (start 428.77 289.33) (end 431.2184 289.33) (width 0.25) (layer F.Cu) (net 33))
 (segment (start 438.2615 281.85) (end 438.25 281.85) (width 0.25) (layer F.Cu) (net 33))
 (segment (start 438.25 281.85) (end 432.9 287.2) (width 0.25) (layer F.Cu) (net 33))
 (segment (start 431.2184 289.33) (end 431.47 289.33) (width 0.25) (layer F.Cu) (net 33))
 (segment (start 432.9 287.9) (end 432.9 287.2) (width 0.25) (layer F.Cu) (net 33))
 (segment (start 431.47 289.33) (end 432.9 287.9) (width 0.25) (layer F.Cu) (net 33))
 (segment (start 440.55 282.35) (end 438.4162 282.35) (width 0.25) (layer F.Cu) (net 34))
 (segment (start 438.4162 282.35) (end 433.698 287.0682) (width 0.25) (layer F.Cu) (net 34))
 (segment (start 433.698 287.0682) (end 433.698 288.212) (width 0.25) (layer F.Cu) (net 34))
 (segment (start 433.698 288.212) (end 431.31 290.6) (width 0.25) (layer F.Cu) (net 34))
 (segment (start 430.04 290.6) (end 431.31 290.6) (width 0.25) (layer F.Cu) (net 34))
 (segment (start 440.55 282.85) (end 438.5637 282.85) (width 0.25) (layer F.Cu) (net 35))
 (segment (start 438.5637 282.85) (end 434.1483 287.2654) (width 0.25) (layer F.Cu) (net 35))
 (segment (start 434.1483 287.2654) (end 434.1483 289.0317) (width 0.25) (layer F.Cu) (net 35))
 (segment (start 434.1483 289.0317) (end 431.31 291.87) (width 0.25) (layer F.Cu) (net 35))
 (segment (start 427.5 293.14) (end 428.77 291.87) (width 0.25) (layer F.Cu) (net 35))
 (segment (start 428.77 291.87) (end 431.31 291.87) (width 0.25) (layer F.Cu) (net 35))
 (segment (start 440.55 283.35) (end 438.7727 283.35) (width 0.25) (layer F.Cu) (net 36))
 (segment (start 438.7727 283.35) (end 435.0489 287.0738) (width 0.25) (layer F.Cu) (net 36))
 (segment (start 435.0489 287.0738) (end 435.0489 289.4011) (width 0.25) (layer F.Cu) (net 36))
 (segment (start 435.0489 289.4011) (end 431.31 293.14) (width 0.25) (layer F.Cu) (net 36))
 (segment (start 430.04 293.14) (end 431.31 293.14) (width 0.25) (layer F.Cu) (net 36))
 (segment (start 440.55 283.85) (end 438.9096 283.85) (width 0.25) (layer F.Cu) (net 37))
 (segment (start 438.9096 283.85) (end 435.4992 287.2604) (width 0.25) (layer F.Cu) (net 37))
 (segment (start 435.4992 287.2604) (end 435.4992 290.2208) (width 0.25) (layer F.Cu) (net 37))
 (segment (start 435.4992 290.2208) (end 431.31 294.41) (width 0.25) (layer F.Cu) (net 37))
 (segment (start 427.5 295.68) (end 428.77 294.41) (width 0.25) (layer F.Cu) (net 37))
 (segment (start 428.77 294.41) (end 431.31 294.41) (width 0.25) (layer F.Cu) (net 37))
 (segment (start 440.55 284.35) (end 439.0465 284.35) (width 0.25) (layer F.Cu) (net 38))
 (segment (start 439.0465 284.35) (end 435.9495 287.447) (width 0.25) (layer F.Cu) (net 38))
 (segment (start 435.9495 287.447) (end 435.9495 291.0405) (width 0.25) (layer F.Cu) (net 38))
 (segment (start 435.9495 291.0405) (end 431.31 295.68) (width 0.25) (layer F.Cu) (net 38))
 (segment (start 430.04 295.68) (end 431.31 295.68) (width 0.25) (layer F.Cu) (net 38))
 (segment (start 440.55 284.85) (end 439.1834 284.85) (width 0.25) (layer F.Cu) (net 39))
 (segment (start 439.1834 284.85) (end 437.3003 286.7331) (width 0.25) (layer F.Cu) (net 39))
 (segment (start 437.3003 286.7331) (end 437.3003 290.9997) (width 0.25) (layer F.Cu) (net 39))
 (segment (start 437.3003 290.9997) (end 431.3 297) (width 0.25) (layer F.Cu) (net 39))
 (segment (start 427.5 298.22) (end 428.72 297) (width 0.25) (layer F.Cu) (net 39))
 (segment (start 428.72 297) (end 431.3 297) (width 0.25) (layer F.Cu) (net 39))
 (segment (start 431.28 298.22) (end 437.7507 291.7493) (width 0.25) (layer F.Cu) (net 40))
 (segment (start 437.7507 291.7493) (end 437.7507 286.9419) (width 0.25) (layer F.Cu) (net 40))
 (segment (start 437.7507 286.9419) (end 439.3426 285.35) (width 0.25) (layer F.Cu) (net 40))
 (segment (start 439.3426 285.35) (end 440.55 285.35) (width 0.25) (layer F.Cu) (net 40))
 (segment (start 430.04 298.22) (end 431.28 298.22) (width 0.25) (layer F.Cu) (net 40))
 (segment (start 431.3 299.5) (end 438.266 292.534) (width 0.25) (layer F.Cu) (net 41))
 (segment (start 438.266 292.534) (end 438.266 287.0712) (width 0.25) (layer F.Cu) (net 41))
 (segment (start 438.266 287.0712) (end 439.4872 285.85) (width 0.25) (layer F.Cu) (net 41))
 (segment (start 439.4872 285.85) (end 440.55 285.85) (width 0.25) (layer F.Cu) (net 41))
 (segment (start 427.5 300.76) (end 428.76 299.5) (width 0.25) (layer F.Cu) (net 41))
 (segment (start 428.76 299.5) (end 431.3 299.5) (width 0.25) (layer F.Cu) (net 41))
 (segment (start 430.04 300.76) (end 432.14 300.76) (width 0.25) (layer F.Cu) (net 42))
 (segment (start 432.14 300.76) (end 439.1 293.8) (width 0.25) (layer F.Cu) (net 42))
 (segment (start 439.1 293.8) (end 439.1 286.9) (width 0.25) (layer F.Cu) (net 42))
 (segment (start 439.1 286.9) (end 439.65 286.35) (width 0.25) (layer F.Cu) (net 42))
 (segment (start 439.65 286.35) (end 440.55 286.35) (width 0.25) (layer F.Cu) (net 42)))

